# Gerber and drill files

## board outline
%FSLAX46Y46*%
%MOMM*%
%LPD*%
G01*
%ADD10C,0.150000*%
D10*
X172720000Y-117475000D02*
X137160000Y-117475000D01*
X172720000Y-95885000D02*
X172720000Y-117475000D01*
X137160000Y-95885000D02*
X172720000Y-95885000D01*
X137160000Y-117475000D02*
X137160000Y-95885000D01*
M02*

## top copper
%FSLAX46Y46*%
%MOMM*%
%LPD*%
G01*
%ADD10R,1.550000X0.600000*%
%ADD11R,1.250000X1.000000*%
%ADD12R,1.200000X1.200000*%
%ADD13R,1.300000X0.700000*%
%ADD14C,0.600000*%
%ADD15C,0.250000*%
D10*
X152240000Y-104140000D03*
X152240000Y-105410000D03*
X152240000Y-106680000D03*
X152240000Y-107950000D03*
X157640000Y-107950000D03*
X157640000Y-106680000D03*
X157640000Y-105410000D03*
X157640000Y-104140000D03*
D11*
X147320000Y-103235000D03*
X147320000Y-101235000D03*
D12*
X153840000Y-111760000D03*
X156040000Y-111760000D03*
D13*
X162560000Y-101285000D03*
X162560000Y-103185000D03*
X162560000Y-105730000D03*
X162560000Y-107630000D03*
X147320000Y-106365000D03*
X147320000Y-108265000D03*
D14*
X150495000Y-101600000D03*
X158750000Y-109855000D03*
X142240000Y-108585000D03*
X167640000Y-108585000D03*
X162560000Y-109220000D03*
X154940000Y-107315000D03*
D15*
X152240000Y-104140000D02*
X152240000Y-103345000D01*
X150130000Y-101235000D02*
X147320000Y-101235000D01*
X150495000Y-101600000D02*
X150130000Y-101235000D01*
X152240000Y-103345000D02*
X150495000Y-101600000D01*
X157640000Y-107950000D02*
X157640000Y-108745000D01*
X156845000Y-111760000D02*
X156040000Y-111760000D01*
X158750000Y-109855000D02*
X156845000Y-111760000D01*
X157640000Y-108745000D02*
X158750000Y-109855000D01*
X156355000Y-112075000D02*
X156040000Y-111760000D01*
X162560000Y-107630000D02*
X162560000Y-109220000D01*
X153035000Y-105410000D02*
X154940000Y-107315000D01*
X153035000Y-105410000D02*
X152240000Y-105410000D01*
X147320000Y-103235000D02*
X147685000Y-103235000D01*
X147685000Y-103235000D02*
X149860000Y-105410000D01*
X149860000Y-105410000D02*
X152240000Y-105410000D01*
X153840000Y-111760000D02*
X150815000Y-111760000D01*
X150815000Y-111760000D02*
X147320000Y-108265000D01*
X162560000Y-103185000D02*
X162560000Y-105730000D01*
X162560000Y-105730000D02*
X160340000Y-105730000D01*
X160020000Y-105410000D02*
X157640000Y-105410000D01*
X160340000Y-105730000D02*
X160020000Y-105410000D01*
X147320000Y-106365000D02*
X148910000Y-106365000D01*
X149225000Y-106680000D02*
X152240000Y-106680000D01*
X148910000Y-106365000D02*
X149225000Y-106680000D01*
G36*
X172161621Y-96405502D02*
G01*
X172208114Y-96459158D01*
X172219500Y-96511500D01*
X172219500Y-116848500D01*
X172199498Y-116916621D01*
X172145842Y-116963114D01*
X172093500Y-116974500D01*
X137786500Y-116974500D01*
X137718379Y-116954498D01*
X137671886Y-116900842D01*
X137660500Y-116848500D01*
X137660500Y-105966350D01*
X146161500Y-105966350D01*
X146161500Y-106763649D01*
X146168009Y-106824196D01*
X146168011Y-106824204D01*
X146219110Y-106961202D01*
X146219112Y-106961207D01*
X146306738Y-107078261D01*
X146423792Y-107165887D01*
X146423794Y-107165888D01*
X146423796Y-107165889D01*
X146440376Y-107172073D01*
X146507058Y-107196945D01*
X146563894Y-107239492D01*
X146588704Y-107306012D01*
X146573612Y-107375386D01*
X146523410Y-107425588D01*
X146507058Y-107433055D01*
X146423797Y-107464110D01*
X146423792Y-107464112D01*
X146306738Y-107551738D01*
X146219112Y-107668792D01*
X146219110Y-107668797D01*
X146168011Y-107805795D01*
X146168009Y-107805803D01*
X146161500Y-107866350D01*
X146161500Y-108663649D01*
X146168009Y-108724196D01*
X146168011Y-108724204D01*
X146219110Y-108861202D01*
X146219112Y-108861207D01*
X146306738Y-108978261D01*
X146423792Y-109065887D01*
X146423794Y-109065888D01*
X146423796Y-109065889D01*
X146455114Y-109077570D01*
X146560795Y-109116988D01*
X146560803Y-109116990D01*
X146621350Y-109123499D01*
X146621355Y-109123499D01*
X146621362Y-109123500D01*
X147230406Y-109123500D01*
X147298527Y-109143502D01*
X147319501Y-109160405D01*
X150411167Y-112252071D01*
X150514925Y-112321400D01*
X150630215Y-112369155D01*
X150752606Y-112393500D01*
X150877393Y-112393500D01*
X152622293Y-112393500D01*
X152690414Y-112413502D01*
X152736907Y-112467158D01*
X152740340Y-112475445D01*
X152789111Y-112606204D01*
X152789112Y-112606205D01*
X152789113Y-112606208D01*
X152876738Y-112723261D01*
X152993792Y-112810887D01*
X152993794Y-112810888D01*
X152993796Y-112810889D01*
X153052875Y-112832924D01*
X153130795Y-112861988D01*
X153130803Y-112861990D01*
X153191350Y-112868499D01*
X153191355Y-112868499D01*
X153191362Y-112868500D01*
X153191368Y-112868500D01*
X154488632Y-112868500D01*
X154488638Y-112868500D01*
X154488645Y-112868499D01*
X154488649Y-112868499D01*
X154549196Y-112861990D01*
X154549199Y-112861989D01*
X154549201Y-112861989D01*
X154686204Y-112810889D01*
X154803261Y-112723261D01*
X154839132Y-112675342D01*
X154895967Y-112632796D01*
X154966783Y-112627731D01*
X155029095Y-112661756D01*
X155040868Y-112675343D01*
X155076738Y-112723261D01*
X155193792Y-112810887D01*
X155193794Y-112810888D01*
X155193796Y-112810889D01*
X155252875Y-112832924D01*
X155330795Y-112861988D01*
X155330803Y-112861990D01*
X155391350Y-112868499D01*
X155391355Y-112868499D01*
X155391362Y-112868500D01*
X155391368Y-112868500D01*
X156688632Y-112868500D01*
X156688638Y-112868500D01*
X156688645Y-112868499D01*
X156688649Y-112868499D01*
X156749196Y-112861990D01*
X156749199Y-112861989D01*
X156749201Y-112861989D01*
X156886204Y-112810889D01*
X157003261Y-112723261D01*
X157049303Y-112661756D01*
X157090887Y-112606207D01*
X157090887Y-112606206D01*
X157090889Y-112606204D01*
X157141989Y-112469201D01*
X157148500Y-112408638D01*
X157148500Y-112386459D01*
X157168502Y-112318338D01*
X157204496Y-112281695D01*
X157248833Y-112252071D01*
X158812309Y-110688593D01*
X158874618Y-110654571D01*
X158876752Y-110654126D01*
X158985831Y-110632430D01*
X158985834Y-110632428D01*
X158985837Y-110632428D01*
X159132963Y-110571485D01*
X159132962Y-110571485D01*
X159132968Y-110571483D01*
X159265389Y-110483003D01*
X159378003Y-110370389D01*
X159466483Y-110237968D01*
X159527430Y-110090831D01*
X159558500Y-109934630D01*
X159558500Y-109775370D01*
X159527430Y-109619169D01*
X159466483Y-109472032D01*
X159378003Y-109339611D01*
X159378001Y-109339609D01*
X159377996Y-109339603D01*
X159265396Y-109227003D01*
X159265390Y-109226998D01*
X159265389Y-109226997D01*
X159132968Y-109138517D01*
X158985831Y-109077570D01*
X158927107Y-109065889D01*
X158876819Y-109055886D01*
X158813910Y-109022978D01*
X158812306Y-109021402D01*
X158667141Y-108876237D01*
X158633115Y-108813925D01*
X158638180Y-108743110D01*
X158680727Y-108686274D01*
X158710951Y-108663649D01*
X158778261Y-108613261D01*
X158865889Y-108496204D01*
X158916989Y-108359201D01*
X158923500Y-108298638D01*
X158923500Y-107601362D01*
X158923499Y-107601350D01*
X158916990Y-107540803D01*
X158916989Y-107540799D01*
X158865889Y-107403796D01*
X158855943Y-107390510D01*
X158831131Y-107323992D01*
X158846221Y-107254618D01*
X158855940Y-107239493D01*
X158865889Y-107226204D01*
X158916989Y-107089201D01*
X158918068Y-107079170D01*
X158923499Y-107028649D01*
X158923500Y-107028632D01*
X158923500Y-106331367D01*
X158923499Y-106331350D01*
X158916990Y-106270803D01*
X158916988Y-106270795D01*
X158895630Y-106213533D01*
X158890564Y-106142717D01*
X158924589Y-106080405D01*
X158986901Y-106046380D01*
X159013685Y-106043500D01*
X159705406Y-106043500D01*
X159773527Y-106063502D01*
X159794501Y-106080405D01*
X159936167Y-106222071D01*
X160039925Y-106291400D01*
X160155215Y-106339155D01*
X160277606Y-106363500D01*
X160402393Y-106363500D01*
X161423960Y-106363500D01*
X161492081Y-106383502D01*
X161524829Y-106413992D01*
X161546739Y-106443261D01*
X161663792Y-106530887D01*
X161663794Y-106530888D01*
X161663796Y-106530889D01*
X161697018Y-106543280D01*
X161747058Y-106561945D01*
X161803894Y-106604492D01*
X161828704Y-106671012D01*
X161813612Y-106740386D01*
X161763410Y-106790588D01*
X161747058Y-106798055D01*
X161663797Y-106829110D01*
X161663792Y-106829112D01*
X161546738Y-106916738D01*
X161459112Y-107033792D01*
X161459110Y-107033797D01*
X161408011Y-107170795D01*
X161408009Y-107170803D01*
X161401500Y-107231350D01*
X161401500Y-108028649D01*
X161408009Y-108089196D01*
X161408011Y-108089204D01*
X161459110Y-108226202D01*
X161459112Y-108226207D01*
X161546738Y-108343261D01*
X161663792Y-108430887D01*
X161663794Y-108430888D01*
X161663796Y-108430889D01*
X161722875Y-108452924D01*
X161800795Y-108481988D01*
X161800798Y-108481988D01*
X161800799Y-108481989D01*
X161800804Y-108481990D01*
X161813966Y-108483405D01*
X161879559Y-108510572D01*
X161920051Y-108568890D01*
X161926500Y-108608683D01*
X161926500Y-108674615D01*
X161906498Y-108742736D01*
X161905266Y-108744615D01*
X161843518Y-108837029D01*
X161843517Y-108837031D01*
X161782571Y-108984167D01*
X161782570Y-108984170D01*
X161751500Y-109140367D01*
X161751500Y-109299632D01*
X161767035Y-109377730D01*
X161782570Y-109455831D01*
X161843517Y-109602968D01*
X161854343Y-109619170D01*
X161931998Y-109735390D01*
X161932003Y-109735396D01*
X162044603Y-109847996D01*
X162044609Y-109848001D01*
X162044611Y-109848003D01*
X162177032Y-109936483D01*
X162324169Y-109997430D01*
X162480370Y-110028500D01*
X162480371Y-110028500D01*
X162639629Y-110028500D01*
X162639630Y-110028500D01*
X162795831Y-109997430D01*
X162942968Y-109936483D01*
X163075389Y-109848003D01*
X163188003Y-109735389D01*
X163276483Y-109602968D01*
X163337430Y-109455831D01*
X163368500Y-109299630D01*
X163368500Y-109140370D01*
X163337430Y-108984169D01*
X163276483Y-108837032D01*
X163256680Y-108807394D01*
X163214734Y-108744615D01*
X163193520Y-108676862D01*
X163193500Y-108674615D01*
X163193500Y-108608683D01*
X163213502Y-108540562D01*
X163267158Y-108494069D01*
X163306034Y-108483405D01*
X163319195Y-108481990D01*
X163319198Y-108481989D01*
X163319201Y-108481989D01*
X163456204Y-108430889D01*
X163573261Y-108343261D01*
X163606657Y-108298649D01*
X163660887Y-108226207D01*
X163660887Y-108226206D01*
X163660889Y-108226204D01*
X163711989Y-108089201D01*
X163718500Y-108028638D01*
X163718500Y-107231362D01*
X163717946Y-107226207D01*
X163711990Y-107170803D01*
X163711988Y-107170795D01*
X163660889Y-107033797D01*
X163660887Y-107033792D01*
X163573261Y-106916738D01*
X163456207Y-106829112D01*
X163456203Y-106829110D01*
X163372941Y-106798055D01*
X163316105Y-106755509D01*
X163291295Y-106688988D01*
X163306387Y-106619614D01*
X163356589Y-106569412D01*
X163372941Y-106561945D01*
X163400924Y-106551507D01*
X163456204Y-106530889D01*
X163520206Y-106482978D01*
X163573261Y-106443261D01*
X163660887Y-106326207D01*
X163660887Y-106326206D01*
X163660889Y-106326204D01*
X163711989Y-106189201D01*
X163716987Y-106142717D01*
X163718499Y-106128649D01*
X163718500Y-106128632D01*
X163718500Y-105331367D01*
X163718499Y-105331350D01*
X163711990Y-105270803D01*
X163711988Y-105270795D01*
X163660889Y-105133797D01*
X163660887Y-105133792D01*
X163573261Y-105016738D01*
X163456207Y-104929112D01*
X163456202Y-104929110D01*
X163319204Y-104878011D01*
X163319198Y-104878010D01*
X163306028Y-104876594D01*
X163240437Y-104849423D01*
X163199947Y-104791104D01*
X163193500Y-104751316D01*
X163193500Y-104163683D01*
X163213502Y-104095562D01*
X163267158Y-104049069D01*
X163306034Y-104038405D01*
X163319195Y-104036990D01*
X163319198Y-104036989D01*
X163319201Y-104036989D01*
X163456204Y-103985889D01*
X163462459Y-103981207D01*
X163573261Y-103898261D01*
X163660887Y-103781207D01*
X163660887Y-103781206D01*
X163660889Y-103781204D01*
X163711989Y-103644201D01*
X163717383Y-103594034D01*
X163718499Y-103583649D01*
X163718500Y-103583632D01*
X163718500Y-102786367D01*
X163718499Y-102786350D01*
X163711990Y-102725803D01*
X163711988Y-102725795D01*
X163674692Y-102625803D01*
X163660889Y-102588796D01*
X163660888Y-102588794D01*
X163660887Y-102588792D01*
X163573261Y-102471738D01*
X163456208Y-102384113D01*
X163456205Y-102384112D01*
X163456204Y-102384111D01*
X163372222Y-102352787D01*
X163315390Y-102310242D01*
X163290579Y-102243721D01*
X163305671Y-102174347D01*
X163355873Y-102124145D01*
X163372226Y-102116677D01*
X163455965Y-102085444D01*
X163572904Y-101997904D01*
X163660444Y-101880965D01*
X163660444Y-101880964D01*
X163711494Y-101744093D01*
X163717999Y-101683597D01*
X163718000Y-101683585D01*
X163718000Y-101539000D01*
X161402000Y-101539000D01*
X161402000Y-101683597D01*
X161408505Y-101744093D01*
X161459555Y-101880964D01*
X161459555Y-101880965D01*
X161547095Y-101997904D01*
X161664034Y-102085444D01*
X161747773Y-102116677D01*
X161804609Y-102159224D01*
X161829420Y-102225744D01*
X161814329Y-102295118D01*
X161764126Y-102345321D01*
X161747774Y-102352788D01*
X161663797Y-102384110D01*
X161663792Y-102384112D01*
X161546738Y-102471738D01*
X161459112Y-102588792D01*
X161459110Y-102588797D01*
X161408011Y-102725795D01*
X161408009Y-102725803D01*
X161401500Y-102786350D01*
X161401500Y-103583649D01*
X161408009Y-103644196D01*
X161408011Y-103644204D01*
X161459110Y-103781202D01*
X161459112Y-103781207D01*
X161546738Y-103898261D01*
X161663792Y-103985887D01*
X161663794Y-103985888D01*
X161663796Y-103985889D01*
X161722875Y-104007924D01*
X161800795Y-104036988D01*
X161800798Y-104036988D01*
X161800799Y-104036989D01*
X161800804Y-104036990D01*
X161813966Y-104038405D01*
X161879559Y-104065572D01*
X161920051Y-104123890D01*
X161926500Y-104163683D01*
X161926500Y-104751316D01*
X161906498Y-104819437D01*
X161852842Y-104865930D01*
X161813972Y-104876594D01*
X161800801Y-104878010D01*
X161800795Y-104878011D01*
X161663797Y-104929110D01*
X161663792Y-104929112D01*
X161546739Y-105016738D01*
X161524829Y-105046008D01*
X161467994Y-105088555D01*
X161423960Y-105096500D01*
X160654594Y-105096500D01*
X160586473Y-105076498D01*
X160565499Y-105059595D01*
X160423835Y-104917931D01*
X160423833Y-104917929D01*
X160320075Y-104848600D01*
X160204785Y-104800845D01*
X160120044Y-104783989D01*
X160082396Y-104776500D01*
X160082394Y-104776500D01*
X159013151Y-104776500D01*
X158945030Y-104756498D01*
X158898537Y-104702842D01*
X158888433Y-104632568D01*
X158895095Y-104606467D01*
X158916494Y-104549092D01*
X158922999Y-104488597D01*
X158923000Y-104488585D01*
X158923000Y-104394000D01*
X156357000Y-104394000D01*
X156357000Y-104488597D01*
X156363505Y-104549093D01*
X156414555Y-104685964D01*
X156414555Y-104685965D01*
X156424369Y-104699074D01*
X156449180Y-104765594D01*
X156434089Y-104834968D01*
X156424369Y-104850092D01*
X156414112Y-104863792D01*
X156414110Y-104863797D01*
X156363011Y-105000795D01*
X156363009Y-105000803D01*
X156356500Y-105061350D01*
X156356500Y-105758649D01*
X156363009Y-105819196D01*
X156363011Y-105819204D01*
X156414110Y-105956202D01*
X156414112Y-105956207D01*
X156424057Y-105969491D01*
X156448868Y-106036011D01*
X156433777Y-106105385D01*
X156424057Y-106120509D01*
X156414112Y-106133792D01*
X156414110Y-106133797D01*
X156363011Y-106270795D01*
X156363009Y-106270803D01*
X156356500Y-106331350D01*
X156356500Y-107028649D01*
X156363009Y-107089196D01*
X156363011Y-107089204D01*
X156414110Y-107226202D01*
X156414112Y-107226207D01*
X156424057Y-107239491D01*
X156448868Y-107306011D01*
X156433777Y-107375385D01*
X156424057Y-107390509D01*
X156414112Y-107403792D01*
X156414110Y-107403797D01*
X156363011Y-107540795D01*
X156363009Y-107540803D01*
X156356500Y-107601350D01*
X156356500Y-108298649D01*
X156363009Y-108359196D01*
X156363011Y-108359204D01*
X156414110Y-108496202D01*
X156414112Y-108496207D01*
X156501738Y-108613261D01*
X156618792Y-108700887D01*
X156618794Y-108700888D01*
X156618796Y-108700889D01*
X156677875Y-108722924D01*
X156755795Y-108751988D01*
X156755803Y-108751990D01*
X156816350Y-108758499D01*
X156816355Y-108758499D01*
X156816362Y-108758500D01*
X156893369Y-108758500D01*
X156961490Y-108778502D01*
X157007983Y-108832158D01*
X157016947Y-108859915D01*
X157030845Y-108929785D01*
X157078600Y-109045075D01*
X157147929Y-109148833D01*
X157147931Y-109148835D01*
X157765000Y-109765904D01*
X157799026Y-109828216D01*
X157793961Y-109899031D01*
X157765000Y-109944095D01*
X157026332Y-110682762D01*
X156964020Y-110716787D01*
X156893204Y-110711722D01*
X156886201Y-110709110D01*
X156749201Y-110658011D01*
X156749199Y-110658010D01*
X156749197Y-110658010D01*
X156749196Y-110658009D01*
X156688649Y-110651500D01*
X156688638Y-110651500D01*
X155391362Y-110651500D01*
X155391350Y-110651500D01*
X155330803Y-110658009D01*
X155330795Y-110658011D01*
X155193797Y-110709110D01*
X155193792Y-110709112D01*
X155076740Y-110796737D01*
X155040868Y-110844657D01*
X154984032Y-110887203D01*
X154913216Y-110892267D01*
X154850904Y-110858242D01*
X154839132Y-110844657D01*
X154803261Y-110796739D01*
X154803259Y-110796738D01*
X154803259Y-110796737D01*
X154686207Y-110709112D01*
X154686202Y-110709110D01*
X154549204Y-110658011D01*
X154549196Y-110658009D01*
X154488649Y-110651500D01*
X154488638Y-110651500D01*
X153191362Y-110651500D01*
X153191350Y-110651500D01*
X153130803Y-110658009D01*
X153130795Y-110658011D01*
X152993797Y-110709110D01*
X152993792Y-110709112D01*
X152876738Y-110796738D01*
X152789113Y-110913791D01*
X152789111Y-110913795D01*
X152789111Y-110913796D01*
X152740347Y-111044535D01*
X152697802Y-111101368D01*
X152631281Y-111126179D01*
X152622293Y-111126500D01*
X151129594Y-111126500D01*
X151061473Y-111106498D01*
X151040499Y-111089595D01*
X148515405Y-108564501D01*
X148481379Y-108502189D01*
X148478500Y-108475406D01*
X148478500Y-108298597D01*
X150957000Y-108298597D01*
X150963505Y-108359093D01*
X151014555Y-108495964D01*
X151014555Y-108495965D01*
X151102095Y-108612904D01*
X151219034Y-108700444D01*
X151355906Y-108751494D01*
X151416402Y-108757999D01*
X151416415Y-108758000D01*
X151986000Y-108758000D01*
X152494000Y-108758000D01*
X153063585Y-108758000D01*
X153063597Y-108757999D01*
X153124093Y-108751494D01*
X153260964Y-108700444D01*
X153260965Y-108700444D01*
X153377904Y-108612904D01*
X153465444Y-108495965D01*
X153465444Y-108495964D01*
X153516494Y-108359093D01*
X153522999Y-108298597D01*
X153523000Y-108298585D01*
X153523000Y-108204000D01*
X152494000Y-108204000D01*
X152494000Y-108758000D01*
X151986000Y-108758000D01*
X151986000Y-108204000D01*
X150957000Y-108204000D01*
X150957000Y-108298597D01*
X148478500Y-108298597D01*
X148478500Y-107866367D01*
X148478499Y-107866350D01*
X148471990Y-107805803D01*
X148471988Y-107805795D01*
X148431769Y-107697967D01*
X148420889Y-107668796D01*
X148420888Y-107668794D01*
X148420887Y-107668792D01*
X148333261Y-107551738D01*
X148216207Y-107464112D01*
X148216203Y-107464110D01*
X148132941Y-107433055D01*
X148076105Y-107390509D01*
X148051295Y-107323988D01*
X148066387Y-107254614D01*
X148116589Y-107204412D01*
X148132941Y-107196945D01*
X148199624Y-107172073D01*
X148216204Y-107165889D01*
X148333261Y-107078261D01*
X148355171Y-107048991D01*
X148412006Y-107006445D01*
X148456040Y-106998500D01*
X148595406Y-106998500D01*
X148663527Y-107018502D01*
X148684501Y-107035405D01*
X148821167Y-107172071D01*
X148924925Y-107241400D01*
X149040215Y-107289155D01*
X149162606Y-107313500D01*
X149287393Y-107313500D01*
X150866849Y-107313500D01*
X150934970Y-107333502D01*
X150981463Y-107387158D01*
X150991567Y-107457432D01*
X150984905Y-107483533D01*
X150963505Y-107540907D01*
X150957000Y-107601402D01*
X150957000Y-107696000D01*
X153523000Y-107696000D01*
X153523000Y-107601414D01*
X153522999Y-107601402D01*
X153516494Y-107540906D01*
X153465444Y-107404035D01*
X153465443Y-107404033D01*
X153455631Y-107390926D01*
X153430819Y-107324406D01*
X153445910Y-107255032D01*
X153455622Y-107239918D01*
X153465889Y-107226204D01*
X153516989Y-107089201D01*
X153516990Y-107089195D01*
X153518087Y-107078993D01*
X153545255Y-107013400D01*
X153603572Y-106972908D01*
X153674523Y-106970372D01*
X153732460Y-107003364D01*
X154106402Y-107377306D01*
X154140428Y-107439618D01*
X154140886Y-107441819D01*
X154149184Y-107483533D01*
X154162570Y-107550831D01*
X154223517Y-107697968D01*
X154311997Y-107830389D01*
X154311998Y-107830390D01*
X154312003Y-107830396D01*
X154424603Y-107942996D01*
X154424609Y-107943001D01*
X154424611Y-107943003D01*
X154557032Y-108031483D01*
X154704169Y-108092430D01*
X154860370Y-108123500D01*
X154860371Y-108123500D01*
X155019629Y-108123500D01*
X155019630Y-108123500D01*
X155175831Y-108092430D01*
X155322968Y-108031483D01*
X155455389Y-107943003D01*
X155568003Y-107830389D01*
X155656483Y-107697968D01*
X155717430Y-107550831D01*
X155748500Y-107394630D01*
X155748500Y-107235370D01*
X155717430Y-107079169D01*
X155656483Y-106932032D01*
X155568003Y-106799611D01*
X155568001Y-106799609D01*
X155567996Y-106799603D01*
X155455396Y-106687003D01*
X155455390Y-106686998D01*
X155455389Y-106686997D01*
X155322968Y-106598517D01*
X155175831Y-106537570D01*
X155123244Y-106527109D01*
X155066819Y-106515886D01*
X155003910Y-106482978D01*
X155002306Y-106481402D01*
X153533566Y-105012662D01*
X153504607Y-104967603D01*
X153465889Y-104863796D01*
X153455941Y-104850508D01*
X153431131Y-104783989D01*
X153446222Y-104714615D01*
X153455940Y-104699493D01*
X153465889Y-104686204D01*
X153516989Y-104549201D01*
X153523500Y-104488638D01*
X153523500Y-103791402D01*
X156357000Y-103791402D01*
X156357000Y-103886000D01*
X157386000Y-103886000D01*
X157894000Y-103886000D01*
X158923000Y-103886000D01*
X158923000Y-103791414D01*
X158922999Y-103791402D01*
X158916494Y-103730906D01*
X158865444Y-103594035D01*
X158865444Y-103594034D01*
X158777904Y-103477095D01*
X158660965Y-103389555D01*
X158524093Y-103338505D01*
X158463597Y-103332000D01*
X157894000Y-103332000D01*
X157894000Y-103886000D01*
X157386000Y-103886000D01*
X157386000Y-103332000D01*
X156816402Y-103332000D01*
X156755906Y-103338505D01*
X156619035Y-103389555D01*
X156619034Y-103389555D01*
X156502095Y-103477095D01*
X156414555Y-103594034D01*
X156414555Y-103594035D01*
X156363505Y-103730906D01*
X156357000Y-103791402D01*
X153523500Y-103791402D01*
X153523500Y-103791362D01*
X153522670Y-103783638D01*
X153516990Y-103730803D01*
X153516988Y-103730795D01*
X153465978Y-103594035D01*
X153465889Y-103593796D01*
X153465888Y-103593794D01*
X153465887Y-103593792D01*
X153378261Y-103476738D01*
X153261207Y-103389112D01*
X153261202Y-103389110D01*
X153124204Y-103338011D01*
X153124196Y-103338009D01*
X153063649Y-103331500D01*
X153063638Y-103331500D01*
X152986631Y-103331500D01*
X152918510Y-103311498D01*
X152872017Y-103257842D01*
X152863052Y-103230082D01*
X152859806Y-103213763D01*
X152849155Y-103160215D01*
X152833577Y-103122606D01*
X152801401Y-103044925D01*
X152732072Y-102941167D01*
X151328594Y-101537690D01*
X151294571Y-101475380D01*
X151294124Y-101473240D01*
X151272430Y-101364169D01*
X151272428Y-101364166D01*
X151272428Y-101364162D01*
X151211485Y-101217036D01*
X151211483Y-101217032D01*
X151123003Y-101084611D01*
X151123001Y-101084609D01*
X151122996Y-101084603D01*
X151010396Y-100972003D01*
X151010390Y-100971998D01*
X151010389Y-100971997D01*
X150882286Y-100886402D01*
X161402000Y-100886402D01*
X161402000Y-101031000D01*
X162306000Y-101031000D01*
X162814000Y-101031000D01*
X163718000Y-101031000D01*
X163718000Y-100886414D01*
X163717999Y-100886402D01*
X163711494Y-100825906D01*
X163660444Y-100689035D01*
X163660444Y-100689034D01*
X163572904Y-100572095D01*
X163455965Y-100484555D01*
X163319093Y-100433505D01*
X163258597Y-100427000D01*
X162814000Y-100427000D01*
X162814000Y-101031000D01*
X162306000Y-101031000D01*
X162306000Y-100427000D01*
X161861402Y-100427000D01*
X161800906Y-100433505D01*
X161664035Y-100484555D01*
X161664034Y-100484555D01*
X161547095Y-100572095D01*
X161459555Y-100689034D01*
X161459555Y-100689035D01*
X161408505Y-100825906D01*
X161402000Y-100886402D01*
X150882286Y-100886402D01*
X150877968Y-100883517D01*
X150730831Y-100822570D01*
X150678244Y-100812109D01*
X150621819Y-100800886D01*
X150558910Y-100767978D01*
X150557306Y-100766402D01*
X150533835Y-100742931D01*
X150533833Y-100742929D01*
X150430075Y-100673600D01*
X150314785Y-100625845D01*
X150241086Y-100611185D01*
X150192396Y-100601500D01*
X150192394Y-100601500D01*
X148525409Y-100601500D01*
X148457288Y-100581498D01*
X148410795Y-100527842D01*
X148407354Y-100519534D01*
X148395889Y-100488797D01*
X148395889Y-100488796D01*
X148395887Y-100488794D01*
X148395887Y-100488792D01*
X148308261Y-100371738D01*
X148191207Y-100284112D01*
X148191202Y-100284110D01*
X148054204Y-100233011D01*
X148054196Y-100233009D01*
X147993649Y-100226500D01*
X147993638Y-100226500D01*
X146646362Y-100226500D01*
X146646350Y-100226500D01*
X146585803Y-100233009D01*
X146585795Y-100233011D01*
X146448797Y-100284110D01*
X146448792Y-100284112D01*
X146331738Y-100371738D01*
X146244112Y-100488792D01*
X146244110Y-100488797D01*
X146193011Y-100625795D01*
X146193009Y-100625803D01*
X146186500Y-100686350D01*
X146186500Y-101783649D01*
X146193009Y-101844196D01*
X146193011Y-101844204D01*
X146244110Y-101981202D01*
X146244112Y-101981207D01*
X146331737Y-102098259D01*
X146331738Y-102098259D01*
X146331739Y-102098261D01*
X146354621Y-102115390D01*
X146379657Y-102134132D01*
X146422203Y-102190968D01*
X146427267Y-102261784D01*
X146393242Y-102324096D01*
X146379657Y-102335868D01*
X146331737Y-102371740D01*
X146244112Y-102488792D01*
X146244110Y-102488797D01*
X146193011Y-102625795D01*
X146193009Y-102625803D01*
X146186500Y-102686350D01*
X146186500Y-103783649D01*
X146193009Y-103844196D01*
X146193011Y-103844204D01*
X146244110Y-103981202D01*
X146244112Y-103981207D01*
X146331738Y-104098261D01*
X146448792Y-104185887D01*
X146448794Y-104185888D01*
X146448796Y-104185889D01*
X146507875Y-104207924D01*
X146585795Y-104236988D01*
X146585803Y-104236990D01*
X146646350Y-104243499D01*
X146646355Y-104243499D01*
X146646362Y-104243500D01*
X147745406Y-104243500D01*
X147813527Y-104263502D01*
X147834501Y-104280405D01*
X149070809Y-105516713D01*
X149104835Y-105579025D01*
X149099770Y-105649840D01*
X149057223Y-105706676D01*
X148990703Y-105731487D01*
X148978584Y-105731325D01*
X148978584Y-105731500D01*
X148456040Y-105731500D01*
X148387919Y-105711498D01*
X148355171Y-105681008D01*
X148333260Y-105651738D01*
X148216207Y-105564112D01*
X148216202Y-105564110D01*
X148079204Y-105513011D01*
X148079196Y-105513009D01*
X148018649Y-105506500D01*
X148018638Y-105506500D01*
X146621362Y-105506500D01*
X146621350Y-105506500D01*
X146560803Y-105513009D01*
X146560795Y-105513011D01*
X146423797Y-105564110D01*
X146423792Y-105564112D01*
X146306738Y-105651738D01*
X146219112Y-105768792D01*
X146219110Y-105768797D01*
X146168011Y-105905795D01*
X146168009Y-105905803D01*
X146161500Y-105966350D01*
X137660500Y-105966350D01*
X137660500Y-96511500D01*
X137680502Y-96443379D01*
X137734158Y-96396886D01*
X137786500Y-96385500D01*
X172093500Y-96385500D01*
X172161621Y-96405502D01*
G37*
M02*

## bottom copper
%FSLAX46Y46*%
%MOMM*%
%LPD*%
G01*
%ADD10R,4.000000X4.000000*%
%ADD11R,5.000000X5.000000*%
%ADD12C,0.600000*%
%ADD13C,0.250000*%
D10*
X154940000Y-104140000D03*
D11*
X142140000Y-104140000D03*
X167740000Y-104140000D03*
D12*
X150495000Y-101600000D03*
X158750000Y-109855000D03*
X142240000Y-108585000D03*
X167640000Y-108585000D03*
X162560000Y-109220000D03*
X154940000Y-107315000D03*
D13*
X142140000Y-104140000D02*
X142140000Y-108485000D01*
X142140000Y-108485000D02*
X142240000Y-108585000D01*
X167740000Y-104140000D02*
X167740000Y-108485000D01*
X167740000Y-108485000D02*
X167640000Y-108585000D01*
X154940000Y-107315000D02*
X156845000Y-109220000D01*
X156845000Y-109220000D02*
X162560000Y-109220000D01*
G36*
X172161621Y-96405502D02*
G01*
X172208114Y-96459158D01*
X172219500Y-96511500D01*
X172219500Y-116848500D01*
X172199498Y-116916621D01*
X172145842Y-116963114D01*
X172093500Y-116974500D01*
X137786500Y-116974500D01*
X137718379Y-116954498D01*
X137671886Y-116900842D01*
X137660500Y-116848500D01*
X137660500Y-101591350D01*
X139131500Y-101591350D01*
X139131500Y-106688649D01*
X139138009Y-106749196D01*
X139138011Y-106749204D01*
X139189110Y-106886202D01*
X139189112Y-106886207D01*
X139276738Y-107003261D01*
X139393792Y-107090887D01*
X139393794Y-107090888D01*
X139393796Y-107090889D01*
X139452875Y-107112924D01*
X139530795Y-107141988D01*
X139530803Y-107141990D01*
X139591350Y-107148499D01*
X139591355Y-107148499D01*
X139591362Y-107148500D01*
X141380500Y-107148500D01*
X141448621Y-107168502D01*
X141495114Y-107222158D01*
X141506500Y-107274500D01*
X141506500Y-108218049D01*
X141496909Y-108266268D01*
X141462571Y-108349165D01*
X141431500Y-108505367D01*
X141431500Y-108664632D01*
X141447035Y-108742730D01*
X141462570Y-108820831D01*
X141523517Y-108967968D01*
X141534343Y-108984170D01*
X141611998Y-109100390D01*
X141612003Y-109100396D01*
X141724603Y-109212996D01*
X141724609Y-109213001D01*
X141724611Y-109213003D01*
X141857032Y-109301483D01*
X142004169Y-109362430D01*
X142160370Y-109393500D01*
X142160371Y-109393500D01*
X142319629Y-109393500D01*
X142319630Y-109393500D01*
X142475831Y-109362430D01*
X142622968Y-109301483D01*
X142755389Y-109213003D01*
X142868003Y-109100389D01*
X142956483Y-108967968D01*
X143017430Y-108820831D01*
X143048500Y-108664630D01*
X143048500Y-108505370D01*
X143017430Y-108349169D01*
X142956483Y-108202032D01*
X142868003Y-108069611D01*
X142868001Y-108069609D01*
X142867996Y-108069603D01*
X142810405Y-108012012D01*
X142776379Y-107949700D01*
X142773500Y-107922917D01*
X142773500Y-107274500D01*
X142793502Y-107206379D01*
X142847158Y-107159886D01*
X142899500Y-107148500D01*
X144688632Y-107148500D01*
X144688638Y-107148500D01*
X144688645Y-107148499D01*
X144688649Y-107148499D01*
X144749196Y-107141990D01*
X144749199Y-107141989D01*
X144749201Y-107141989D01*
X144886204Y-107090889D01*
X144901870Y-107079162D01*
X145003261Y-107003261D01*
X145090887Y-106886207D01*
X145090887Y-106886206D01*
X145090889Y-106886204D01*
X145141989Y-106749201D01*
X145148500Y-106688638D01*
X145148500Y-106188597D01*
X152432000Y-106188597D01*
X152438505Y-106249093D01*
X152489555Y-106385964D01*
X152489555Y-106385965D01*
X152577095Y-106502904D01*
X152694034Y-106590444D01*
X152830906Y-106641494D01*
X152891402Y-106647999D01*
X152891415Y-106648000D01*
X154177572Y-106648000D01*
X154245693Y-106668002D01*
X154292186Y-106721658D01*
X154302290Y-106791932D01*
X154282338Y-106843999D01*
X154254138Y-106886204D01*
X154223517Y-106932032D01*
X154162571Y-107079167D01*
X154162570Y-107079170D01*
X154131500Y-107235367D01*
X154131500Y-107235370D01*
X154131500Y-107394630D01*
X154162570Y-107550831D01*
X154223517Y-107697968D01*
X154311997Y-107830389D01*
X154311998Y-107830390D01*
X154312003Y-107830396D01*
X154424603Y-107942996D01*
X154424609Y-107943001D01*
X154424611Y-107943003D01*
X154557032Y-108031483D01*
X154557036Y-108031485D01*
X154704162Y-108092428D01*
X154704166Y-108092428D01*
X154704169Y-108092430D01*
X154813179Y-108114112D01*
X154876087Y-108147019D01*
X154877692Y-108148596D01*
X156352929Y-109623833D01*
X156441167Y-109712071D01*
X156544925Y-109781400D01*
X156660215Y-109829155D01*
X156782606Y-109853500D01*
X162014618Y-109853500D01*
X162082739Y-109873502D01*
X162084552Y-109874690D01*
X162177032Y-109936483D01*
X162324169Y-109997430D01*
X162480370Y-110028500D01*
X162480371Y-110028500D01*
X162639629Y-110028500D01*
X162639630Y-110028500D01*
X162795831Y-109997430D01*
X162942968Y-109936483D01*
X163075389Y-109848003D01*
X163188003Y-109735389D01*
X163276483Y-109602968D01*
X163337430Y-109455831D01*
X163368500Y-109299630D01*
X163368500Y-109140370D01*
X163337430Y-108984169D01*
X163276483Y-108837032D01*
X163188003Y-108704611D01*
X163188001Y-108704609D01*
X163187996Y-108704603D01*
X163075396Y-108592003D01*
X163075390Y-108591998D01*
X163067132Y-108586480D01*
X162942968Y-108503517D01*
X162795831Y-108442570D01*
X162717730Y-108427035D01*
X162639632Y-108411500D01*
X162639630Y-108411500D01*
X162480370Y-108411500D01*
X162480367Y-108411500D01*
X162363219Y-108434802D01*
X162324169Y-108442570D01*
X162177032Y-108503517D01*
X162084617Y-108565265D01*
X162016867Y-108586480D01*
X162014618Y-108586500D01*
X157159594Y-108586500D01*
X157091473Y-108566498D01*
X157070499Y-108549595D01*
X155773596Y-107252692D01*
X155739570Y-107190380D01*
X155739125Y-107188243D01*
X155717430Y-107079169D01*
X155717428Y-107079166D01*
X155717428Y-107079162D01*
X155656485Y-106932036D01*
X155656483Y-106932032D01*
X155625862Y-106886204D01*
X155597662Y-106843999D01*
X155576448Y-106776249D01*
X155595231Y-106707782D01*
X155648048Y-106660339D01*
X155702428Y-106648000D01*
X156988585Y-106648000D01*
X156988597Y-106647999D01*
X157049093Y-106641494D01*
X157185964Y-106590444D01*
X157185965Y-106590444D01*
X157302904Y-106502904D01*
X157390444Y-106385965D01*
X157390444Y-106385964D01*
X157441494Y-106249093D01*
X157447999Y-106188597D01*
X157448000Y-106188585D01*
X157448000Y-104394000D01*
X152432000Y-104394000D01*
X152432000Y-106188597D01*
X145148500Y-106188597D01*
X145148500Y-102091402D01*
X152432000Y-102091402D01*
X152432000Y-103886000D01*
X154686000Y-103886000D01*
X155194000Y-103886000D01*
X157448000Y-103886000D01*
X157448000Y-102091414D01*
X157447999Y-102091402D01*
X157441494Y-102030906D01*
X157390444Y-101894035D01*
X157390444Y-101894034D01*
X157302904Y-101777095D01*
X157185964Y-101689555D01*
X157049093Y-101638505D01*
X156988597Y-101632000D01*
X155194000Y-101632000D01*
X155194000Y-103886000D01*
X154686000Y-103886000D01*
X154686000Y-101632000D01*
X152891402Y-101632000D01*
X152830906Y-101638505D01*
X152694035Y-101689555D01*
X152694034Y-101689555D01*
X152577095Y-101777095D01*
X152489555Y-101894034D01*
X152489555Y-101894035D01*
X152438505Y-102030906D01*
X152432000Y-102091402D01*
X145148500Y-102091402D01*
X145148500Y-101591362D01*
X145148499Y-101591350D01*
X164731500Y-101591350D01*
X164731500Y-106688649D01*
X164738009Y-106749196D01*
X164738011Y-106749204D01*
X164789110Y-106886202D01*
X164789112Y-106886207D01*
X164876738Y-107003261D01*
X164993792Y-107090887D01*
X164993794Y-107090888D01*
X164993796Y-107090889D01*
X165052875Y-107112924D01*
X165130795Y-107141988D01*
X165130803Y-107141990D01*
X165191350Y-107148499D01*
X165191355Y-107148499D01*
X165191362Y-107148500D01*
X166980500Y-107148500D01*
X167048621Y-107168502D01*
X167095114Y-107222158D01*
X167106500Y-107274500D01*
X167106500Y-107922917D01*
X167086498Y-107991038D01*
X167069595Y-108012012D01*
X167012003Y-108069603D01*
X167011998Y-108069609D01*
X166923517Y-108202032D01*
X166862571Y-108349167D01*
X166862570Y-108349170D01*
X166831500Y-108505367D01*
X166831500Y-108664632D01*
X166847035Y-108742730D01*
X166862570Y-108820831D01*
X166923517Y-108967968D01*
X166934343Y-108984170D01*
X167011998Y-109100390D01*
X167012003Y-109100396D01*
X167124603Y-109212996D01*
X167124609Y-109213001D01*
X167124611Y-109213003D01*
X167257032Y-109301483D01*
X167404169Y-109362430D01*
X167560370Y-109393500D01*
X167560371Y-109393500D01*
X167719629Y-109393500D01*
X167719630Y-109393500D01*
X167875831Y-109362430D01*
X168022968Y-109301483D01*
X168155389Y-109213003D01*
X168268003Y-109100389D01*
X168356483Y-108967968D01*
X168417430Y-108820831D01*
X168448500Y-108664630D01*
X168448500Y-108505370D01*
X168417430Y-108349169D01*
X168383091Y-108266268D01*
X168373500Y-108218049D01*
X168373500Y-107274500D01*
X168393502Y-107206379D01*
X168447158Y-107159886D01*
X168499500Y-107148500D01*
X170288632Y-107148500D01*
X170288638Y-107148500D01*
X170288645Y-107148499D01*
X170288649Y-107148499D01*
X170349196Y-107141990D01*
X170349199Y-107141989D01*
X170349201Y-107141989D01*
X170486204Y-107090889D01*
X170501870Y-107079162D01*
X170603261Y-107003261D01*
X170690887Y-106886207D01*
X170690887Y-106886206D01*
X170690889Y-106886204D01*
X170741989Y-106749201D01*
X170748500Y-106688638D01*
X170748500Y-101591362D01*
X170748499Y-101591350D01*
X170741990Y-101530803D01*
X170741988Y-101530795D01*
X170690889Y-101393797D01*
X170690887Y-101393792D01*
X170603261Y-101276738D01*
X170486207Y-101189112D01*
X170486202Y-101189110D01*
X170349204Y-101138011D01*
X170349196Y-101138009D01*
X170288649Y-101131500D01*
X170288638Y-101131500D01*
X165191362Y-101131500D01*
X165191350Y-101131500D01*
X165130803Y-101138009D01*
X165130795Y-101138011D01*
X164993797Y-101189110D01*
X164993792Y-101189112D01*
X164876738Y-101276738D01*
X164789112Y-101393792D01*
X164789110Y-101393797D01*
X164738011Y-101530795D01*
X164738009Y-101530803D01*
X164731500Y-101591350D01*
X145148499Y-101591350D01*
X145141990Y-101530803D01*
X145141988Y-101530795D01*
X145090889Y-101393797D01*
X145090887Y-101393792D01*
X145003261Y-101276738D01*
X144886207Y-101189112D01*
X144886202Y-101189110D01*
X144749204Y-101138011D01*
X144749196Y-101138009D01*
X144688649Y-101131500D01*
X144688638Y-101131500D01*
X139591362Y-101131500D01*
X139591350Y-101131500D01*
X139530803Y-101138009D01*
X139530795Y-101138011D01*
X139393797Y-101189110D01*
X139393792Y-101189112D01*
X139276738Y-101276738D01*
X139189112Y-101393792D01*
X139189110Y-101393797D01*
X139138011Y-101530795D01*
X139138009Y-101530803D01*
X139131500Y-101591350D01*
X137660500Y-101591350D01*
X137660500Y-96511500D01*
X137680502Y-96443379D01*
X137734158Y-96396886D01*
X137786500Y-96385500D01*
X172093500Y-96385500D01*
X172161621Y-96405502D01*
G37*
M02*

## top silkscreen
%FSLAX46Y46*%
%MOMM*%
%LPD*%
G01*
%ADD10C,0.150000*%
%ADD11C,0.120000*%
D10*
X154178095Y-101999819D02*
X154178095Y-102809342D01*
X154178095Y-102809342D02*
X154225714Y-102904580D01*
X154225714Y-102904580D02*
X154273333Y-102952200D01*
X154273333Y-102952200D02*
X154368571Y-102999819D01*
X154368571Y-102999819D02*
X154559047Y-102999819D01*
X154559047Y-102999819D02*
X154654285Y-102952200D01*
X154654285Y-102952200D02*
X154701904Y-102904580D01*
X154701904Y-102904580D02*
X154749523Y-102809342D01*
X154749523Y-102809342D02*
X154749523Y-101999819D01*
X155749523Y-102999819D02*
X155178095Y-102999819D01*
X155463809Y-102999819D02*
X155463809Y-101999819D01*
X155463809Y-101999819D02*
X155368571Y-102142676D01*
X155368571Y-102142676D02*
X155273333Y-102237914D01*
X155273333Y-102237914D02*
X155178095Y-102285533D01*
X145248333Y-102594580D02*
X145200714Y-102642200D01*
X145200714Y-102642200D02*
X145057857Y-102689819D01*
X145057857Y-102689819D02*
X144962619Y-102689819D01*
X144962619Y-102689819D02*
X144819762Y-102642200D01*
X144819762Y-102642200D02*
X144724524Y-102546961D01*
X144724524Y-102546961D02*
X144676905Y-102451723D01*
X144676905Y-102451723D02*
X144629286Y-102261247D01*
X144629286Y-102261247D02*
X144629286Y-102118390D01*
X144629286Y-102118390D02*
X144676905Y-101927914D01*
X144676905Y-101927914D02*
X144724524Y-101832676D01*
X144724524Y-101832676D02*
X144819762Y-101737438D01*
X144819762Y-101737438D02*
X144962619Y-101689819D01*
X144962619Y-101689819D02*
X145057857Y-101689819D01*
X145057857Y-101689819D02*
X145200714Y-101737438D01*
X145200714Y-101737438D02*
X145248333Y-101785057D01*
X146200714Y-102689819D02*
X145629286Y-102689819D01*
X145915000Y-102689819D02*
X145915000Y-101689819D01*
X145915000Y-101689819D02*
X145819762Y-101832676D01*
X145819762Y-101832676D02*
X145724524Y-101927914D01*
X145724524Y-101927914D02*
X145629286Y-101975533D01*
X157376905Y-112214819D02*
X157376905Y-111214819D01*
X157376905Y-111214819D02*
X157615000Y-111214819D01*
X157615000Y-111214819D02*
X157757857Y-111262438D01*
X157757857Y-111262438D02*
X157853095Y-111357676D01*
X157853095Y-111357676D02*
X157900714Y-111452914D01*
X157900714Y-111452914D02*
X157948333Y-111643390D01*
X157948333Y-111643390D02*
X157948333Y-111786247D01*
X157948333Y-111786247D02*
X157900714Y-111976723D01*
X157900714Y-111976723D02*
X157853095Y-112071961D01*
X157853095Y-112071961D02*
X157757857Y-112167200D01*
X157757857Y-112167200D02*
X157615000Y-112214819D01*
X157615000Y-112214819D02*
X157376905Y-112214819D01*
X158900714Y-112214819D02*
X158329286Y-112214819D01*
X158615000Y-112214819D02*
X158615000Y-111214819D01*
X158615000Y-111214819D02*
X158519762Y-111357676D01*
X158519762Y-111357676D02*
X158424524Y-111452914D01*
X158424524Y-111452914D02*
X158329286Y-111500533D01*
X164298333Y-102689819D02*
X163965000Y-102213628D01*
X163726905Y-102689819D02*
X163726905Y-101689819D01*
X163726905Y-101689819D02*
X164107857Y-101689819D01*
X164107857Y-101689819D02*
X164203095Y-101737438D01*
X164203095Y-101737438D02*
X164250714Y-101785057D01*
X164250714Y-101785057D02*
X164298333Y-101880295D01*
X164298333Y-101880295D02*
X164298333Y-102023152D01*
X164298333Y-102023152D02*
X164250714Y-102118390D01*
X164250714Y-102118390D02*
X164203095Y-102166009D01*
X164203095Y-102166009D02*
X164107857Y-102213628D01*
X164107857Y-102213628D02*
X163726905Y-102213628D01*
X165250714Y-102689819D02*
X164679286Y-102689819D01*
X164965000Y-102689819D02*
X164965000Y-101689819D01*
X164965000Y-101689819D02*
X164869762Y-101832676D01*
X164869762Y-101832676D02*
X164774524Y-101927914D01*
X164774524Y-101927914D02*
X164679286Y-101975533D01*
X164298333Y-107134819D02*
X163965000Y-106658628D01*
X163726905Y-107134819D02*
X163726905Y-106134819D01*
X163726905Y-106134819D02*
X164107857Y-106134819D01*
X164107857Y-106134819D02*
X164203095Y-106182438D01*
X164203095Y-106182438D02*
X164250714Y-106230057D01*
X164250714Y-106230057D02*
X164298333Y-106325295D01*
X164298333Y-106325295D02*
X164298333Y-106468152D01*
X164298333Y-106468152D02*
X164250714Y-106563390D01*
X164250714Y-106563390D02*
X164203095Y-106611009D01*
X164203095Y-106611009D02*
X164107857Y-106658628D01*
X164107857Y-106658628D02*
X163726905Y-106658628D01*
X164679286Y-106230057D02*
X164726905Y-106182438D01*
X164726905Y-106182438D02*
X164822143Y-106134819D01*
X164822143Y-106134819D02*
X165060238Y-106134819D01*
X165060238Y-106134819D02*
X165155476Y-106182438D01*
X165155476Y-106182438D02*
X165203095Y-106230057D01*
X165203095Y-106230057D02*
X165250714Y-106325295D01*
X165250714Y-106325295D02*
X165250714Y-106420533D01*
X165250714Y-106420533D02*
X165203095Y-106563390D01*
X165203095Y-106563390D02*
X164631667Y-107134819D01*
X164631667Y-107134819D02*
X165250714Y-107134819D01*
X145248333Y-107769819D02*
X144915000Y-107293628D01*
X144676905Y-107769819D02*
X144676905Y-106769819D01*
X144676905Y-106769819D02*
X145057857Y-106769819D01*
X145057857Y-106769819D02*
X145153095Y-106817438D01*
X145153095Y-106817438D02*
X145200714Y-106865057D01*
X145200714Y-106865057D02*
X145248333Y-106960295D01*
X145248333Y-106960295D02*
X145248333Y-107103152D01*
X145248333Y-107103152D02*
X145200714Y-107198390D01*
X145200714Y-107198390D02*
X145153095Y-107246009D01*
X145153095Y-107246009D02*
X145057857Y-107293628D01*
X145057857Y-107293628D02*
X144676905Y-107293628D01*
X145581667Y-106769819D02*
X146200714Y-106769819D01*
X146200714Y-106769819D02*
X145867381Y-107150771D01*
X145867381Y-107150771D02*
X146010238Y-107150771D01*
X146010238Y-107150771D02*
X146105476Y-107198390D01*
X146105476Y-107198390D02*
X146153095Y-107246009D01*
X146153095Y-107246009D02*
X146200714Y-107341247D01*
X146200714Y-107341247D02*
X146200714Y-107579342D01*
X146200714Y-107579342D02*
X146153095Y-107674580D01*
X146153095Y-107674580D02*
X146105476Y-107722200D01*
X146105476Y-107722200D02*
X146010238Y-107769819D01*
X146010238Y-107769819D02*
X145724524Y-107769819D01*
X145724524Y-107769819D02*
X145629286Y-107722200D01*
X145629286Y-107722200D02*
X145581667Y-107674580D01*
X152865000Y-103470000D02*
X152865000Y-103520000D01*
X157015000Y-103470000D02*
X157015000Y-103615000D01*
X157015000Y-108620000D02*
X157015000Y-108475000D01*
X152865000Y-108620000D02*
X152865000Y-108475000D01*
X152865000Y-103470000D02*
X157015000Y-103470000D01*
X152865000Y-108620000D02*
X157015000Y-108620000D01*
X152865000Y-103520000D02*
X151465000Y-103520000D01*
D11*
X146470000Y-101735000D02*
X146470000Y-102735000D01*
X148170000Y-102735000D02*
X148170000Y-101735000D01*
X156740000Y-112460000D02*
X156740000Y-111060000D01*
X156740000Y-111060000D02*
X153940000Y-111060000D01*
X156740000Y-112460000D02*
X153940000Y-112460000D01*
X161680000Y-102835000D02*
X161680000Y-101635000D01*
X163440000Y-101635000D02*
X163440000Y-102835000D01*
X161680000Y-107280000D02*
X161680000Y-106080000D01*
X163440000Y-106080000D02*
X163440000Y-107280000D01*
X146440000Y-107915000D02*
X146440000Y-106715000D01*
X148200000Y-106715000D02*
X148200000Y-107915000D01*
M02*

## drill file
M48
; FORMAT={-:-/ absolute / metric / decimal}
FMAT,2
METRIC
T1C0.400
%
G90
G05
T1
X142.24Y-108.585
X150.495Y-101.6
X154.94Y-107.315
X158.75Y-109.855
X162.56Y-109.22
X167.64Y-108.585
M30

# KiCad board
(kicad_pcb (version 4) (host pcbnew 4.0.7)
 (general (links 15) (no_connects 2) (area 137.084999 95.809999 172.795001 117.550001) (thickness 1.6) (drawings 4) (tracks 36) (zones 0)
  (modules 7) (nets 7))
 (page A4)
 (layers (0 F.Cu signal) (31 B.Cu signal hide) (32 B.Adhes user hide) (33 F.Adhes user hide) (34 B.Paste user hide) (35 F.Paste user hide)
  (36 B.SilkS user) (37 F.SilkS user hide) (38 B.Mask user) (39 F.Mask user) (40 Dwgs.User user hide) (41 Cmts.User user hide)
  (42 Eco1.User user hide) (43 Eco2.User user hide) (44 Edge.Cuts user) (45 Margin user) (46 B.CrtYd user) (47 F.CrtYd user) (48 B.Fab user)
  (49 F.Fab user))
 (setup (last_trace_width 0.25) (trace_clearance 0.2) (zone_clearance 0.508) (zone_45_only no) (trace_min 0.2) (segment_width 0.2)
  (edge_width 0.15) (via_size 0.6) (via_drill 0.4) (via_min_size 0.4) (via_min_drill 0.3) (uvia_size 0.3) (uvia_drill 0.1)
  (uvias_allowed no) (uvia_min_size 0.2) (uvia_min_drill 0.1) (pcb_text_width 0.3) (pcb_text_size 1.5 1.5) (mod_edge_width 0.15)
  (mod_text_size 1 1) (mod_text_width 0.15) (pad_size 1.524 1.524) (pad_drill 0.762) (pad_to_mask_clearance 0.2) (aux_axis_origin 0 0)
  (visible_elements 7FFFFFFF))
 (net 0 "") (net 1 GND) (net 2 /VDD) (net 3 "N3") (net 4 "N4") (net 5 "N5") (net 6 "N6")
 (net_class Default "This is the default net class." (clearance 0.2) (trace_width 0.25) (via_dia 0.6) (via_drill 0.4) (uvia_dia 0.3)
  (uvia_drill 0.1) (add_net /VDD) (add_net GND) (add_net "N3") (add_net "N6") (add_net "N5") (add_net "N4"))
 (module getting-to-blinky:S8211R (layer B.Cu) (at 154.94 104.14)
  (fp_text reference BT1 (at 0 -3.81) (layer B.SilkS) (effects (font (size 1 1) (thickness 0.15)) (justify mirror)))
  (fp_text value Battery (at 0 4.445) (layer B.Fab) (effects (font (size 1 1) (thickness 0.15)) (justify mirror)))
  (pad 2 smd rect (at 0 0) (size 4 4) (layers B.Cu B.Paste B.Mask) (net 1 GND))
  (pad 1 smd rect (at -12.8 0) (size 5 5) (layers B.Cu B.Paste B.Mask) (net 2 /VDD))
  (pad 1 smd rect (at 12.8 0) (size 5 5) (layers B.Cu B.Paste B.Mask) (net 2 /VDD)))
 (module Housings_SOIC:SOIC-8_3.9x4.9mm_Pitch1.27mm (layer F.Cu) (at 154.94 106.045)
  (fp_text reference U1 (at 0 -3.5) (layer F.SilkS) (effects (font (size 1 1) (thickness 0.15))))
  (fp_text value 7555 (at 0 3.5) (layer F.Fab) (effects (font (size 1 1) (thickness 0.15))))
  (fp_line (start -2.075 -2.575) (end -2.075 -2.525) (layer F.SilkS) (width 0.15))
  (fp_line (start 2.075 -2.575) (end 2.075 -2.43) (layer F.SilkS) (width 0.15))
  (fp_line (start 2.075 2.575) (end 2.075 2.43) (layer F.SilkS) (width 0.15))
  (fp_line (start -2.075 2.575) (end -2.075 2.43) (layer F.SilkS) (width 0.15))
  (fp_line (start -2.075 -2.575) (end 2.075 -2.575) (layer F.SilkS) (width 0.15))
  (fp_line (start -2.075 2.575) (end 2.075 2.575) (layer F.SilkS) (width 0.15))
  (fp_line (start -2.075 -2.525) (end -3.475 -2.525) (layer F.SilkS) (width 0.15))
  (pad 1 smd rect (at -2.7 -1.905) (size 1.55 0.6) (layers F.Cu F.Paste F.Mask) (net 1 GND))
  (pad 2 smd rect (at -2.7 -0.635) (size 1.55 0.6) (layers F.Cu F.Paste F.Mask) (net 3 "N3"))
  (pad 3 smd rect (at -2.7 0.635) (size 1.55 0.6) (layers F.Cu F.Paste F.Mask) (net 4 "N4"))
  (pad 4 smd rect (at -2.7 1.905) (size 1.55 0.6) (layers F.Cu F.Paste F.Mask) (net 2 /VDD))
  (pad 5 smd rect (at 2.7 1.905) (size 1.55 0.6) (layers F.Cu F.Paste F.Mask) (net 1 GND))
  (pad 6 smd rect (at 2.7 0.635) (size 1.55 0.6) (layers F.Cu F.Paste F.Mask) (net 3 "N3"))
  (pad 7 smd rect (at 2.7 -0.635) (size 1.55 0.6) (layers F.Cu F.Paste F.Mask) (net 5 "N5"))
  (pad 8 smd rect (at 2.7 -1.905) (size 1.55 0.6) (layers F.Cu F.Paste F.Mask) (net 2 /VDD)))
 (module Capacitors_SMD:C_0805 (layer F.Cu) (at 147.32 102.235 90)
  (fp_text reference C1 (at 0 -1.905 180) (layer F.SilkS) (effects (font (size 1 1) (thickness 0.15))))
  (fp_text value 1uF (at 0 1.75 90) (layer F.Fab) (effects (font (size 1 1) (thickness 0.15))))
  (fp_line (start 0.5 -0.85) (end -0.5 -0.85) (layer F.SilkS) (width 0.12))
  (fp_line (start -0.5 0.85) (end 0.5 0.85) (layer F.SilkS) (width 0.12))
  (pad 1 smd rect (at -1 0 90) (size 1 1.25) (layers F.Cu F.Paste F.Mask) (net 3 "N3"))
  (pad 2 smd rect (at 1 0 90) (size 1 1.25) (layers F.Cu F.Paste F.Mask) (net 1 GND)))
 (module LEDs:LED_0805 (layer F.Cu) (at 154.94 111.76 180)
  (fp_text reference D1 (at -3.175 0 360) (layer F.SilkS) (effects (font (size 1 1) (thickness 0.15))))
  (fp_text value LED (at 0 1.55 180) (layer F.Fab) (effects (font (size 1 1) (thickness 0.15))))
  (fp_line (start -1.8 -0.7) (end -1.8 0.7) (layer F.SilkS) (width 0.12))
  (fp_line (start -1.8 0.7) (end 1 0.7) (layer F.SilkS) (width 0.12))
  (fp_line (start -1.8 -0.7) (end 1 -0.7) (layer F.SilkS) (width 0.12))
  (pad 2 smd rect (at 1.1 0) (size 1.2 1.2) (layers F.Cu F.Paste F.Mask) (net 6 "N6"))
  (pad 1 smd rect (at -1.1 0) (size 1.2 1.2) (layers F.Cu F.Paste F.Mask) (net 1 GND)))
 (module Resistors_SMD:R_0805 (layer F.Cu) (at 162.56 102.235 270)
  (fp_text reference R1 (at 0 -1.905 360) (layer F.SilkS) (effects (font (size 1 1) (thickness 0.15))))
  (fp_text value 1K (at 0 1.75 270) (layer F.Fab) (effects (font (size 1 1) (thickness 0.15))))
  (fp_line (start 0.6 0.88) (end -0.6 0.88) (layer F.SilkS) (width 0.12))
  (fp_line (start -0.6 -0.88) (end 0.6 -0.88) (layer F.SilkS) (width 0.12))
  (pad 1 smd rect (at -0.95 0 270) (size 0.7 1.3) (layers F.Cu F.Paste F.Mask) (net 2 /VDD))
  (pad 2 smd rect (at 0.95 0 270) (size 0.7 1.3) (layers F.Cu F.Paste F.Mask) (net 5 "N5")))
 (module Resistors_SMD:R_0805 (layer F.Cu) (at 162.56 106.68 270)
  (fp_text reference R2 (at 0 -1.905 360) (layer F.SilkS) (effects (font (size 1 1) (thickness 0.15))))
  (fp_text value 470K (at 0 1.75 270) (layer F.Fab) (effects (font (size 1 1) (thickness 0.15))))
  (fp_line (start 0.6 0.88) (end -0.6 0.88) (layer F.SilkS) (width 0.12))
  (fp_line (start -0.6 -0.88) (end 0.6 -0.88) (layer F.SilkS) (width 0.12))
  (pad 1 smd rect (at -0.95 0 270) (size 0.7 1.3) (layers F.Cu F.Paste F.Mask) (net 5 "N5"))
  (pad 2 smd rect (at 0.95 0 270) (size 0.7 1.3) (layers F.Cu F.Paste F.Mask) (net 3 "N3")))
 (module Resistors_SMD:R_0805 (layer F.Cu) (at 147.32 107.315 270)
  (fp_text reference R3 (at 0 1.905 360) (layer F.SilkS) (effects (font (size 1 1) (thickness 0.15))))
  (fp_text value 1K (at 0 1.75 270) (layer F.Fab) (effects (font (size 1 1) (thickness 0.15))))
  (fp_line (start 0.6 0.88) (end -0.6 0.88) (layer F.SilkS) (width 0.12))
  (fp_line (start -0.6 -0.88) (end 0.6 -0.88) (layer F.SilkS) (width 0.12))
  (pad 1 smd rect (at -0.95 0 270) (size 0.7 1.3) (layers F.Cu F.Paste F.Mask) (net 4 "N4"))
  (pad 2 smd rect (at 0.95 0 270) (size 0.7 1.3) (layers F.Cu F.Paste F.Mask) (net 6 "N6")))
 (gr_line (start 172.72 117.475) (end 137.16 117.475) (angle 90) (layer Edge.Cuts) (width 0.15))
 (gr_line (start 172.72 95.885) (end 172.72 117.475) (angle 90) (layer Edge.Cuts) (width 0.15))
 (gr_line (start 137.16 95.885) (end 172.72 95.885) (angle 90) (layer Edge.Cuts) (width 0.15))
 (gr_line (start 137.16 117.475) (end 137.16 95.885) (angle 90) (layer Edge.Cuts) (width 0.15))
 (segment (start 152.24 104.14) (end 152.24 103.345) (width 0.25) (layer F.Cu) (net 1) (status 400000))
 (segment (start 150.13 101.235) (end 147.32 101.235) (width 0.25) (layer F.Cu) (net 1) (status 800000))
 (segment (start 150.495 101.6) (end 150.13 101.235) (width 0.25) (layer F.Cu) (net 1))
 (via (at 150.495 101.6) (size 0.6) (drill 0.4) (layers F.Cu B.Cu) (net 1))
 (segment (start 152.24 103.345) (end 150.495 101.6) (width 0.25) (layer F.Cu) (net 1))
 (segment (start 157.64 107.95) (end 157.64 108.745) (width 0.25) (layer F.Cu) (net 1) (status 400000))
 (segment (start 156.845 111.76) (end 156.04 111.76) (width 0.25) (layer F.Cu) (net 1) (status 800000))
 (segment (start 158.75 109.855) (end 156.845 111.76) (width 0.25) (layer F.Cu) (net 1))
 (via (at 158.75 109.855) (size 0.6) (drill 0.4) (layers F.Cu B.Cu) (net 1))
 (segment (start 157.64 108.745) (end 158.75 109.855) (width 0.25) (layer F.Cu) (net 1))
 (segment (start 156.355 112.075) (end 156.04 111.76) (width 0.25) (layer F.Cu) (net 1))
 (segment (start 142.14 104.14) (end 142.14 108.485) (width 0.25) (layer B.Cu) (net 2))
 (via (at 142.24 108.585) (size 0.6) (drill 0.4) (layers F.Cu B.Cu) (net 2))
 (segment (start 142.14 108.485) (end 142.24 108.585) (width 0.25) (layer B.Cu) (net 2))
 (segment (start 167.74 104.14) (end 167.74 108.485) (width 0.25) (layer B.Cu) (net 2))
 (via (at 167.64 108.585) (size 0.6) (drill 0.4) (layers F.Cu B.Cu) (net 2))
 (segment (start 167.74 108.485) (end 167.64 108.585) (width 0.25) (layer B.Cu) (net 2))
 (segment (start 154.94 107.315) (end 156.845 109.22) (width 0.25) (layer B.Cu) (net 3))
 (via (at 162.56 109.22) (size 0.6) (drill 0.4) (layers F.Cu B.Cu) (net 3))
 (segment (start 162.56 107.63) (end 162.56 109.22) (width 0.25) (layer F.Cu) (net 3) (status 400000))
 (segment (start 153.035 105.41) (end 154.94 107.315) (width 0.25) (layer F.Cu) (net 3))
 (via (at 154.94 107.315) (size 0.6) (drill 0.4) (layers F.Cu B.Cu) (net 3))
 (segment (start 153.035 105.41) (end 152.24 105.41) (width 0.25) (layer F.Cu) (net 3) (status 800000))
 (segment (start 156.845 109.22) (end 162.56 109.22) (width 0.25) (layer B.Cu) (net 3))
 (segment (start 147.32 103.235) (end 147.685 103.235) (width 0.25) (layer F.Cu) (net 3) (status C00000))
 (segment (start 147.685 103.235) (end 149.86 105.41) (width 0.25) (layer F.Cu) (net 3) (status 400000))
 (segment (start 149.86 105.41) (end 152.24 105.41) (width 0.25) (layer F.Cu) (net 3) (status 800000))
 (segment (start 153.84 111.76) (end 150.815 111.76) (width 0.25) (layer F.Cu) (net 6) (status 400000))
 (segment (start 150.815 111.76) (end 147.32 108.265) (width 0.25) (layer F.Cu) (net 6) (status 800000))
 (segment (start 162.56 103.185) (end 162.56 105.73) (width 0.25) (layer F.Cu) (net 5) (status C00000))
 (segment (start 162.56 105.73) (end 160.34 105.73) (width 0.25) (layer F.Cu) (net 5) (status 400000))
 (segment (start 160.02 105.41) (end 157.64 105.41) (width 0.25) (layer F.Cu) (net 5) (status 800000))
 (segment (start 160.34 105.73) (end 160.02 105.41) (width 0.25) (layer F.Cu) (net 5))
 (segment (start 147.32 106.365) (end 148.91 106.365) (width 0.25) (layer F.Cu) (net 4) (status 400000))
 (segment (start 149.225 106.68) (end 152.24 106.68) (width 0.25) (layer F.Cu) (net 4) (status 800000))
 (segment (start 148.91 106.365) (end 149.225 106.68) (width 0.25) (layer F.Cu) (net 4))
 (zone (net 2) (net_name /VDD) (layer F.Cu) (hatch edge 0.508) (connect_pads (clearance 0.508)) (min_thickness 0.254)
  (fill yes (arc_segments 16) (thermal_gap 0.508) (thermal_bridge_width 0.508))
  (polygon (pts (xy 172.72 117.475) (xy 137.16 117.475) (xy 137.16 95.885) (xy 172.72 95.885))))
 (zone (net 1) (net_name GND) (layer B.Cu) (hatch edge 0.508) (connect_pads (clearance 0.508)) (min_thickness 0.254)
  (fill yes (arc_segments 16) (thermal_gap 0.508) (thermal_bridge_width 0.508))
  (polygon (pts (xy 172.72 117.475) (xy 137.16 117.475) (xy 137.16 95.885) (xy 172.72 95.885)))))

